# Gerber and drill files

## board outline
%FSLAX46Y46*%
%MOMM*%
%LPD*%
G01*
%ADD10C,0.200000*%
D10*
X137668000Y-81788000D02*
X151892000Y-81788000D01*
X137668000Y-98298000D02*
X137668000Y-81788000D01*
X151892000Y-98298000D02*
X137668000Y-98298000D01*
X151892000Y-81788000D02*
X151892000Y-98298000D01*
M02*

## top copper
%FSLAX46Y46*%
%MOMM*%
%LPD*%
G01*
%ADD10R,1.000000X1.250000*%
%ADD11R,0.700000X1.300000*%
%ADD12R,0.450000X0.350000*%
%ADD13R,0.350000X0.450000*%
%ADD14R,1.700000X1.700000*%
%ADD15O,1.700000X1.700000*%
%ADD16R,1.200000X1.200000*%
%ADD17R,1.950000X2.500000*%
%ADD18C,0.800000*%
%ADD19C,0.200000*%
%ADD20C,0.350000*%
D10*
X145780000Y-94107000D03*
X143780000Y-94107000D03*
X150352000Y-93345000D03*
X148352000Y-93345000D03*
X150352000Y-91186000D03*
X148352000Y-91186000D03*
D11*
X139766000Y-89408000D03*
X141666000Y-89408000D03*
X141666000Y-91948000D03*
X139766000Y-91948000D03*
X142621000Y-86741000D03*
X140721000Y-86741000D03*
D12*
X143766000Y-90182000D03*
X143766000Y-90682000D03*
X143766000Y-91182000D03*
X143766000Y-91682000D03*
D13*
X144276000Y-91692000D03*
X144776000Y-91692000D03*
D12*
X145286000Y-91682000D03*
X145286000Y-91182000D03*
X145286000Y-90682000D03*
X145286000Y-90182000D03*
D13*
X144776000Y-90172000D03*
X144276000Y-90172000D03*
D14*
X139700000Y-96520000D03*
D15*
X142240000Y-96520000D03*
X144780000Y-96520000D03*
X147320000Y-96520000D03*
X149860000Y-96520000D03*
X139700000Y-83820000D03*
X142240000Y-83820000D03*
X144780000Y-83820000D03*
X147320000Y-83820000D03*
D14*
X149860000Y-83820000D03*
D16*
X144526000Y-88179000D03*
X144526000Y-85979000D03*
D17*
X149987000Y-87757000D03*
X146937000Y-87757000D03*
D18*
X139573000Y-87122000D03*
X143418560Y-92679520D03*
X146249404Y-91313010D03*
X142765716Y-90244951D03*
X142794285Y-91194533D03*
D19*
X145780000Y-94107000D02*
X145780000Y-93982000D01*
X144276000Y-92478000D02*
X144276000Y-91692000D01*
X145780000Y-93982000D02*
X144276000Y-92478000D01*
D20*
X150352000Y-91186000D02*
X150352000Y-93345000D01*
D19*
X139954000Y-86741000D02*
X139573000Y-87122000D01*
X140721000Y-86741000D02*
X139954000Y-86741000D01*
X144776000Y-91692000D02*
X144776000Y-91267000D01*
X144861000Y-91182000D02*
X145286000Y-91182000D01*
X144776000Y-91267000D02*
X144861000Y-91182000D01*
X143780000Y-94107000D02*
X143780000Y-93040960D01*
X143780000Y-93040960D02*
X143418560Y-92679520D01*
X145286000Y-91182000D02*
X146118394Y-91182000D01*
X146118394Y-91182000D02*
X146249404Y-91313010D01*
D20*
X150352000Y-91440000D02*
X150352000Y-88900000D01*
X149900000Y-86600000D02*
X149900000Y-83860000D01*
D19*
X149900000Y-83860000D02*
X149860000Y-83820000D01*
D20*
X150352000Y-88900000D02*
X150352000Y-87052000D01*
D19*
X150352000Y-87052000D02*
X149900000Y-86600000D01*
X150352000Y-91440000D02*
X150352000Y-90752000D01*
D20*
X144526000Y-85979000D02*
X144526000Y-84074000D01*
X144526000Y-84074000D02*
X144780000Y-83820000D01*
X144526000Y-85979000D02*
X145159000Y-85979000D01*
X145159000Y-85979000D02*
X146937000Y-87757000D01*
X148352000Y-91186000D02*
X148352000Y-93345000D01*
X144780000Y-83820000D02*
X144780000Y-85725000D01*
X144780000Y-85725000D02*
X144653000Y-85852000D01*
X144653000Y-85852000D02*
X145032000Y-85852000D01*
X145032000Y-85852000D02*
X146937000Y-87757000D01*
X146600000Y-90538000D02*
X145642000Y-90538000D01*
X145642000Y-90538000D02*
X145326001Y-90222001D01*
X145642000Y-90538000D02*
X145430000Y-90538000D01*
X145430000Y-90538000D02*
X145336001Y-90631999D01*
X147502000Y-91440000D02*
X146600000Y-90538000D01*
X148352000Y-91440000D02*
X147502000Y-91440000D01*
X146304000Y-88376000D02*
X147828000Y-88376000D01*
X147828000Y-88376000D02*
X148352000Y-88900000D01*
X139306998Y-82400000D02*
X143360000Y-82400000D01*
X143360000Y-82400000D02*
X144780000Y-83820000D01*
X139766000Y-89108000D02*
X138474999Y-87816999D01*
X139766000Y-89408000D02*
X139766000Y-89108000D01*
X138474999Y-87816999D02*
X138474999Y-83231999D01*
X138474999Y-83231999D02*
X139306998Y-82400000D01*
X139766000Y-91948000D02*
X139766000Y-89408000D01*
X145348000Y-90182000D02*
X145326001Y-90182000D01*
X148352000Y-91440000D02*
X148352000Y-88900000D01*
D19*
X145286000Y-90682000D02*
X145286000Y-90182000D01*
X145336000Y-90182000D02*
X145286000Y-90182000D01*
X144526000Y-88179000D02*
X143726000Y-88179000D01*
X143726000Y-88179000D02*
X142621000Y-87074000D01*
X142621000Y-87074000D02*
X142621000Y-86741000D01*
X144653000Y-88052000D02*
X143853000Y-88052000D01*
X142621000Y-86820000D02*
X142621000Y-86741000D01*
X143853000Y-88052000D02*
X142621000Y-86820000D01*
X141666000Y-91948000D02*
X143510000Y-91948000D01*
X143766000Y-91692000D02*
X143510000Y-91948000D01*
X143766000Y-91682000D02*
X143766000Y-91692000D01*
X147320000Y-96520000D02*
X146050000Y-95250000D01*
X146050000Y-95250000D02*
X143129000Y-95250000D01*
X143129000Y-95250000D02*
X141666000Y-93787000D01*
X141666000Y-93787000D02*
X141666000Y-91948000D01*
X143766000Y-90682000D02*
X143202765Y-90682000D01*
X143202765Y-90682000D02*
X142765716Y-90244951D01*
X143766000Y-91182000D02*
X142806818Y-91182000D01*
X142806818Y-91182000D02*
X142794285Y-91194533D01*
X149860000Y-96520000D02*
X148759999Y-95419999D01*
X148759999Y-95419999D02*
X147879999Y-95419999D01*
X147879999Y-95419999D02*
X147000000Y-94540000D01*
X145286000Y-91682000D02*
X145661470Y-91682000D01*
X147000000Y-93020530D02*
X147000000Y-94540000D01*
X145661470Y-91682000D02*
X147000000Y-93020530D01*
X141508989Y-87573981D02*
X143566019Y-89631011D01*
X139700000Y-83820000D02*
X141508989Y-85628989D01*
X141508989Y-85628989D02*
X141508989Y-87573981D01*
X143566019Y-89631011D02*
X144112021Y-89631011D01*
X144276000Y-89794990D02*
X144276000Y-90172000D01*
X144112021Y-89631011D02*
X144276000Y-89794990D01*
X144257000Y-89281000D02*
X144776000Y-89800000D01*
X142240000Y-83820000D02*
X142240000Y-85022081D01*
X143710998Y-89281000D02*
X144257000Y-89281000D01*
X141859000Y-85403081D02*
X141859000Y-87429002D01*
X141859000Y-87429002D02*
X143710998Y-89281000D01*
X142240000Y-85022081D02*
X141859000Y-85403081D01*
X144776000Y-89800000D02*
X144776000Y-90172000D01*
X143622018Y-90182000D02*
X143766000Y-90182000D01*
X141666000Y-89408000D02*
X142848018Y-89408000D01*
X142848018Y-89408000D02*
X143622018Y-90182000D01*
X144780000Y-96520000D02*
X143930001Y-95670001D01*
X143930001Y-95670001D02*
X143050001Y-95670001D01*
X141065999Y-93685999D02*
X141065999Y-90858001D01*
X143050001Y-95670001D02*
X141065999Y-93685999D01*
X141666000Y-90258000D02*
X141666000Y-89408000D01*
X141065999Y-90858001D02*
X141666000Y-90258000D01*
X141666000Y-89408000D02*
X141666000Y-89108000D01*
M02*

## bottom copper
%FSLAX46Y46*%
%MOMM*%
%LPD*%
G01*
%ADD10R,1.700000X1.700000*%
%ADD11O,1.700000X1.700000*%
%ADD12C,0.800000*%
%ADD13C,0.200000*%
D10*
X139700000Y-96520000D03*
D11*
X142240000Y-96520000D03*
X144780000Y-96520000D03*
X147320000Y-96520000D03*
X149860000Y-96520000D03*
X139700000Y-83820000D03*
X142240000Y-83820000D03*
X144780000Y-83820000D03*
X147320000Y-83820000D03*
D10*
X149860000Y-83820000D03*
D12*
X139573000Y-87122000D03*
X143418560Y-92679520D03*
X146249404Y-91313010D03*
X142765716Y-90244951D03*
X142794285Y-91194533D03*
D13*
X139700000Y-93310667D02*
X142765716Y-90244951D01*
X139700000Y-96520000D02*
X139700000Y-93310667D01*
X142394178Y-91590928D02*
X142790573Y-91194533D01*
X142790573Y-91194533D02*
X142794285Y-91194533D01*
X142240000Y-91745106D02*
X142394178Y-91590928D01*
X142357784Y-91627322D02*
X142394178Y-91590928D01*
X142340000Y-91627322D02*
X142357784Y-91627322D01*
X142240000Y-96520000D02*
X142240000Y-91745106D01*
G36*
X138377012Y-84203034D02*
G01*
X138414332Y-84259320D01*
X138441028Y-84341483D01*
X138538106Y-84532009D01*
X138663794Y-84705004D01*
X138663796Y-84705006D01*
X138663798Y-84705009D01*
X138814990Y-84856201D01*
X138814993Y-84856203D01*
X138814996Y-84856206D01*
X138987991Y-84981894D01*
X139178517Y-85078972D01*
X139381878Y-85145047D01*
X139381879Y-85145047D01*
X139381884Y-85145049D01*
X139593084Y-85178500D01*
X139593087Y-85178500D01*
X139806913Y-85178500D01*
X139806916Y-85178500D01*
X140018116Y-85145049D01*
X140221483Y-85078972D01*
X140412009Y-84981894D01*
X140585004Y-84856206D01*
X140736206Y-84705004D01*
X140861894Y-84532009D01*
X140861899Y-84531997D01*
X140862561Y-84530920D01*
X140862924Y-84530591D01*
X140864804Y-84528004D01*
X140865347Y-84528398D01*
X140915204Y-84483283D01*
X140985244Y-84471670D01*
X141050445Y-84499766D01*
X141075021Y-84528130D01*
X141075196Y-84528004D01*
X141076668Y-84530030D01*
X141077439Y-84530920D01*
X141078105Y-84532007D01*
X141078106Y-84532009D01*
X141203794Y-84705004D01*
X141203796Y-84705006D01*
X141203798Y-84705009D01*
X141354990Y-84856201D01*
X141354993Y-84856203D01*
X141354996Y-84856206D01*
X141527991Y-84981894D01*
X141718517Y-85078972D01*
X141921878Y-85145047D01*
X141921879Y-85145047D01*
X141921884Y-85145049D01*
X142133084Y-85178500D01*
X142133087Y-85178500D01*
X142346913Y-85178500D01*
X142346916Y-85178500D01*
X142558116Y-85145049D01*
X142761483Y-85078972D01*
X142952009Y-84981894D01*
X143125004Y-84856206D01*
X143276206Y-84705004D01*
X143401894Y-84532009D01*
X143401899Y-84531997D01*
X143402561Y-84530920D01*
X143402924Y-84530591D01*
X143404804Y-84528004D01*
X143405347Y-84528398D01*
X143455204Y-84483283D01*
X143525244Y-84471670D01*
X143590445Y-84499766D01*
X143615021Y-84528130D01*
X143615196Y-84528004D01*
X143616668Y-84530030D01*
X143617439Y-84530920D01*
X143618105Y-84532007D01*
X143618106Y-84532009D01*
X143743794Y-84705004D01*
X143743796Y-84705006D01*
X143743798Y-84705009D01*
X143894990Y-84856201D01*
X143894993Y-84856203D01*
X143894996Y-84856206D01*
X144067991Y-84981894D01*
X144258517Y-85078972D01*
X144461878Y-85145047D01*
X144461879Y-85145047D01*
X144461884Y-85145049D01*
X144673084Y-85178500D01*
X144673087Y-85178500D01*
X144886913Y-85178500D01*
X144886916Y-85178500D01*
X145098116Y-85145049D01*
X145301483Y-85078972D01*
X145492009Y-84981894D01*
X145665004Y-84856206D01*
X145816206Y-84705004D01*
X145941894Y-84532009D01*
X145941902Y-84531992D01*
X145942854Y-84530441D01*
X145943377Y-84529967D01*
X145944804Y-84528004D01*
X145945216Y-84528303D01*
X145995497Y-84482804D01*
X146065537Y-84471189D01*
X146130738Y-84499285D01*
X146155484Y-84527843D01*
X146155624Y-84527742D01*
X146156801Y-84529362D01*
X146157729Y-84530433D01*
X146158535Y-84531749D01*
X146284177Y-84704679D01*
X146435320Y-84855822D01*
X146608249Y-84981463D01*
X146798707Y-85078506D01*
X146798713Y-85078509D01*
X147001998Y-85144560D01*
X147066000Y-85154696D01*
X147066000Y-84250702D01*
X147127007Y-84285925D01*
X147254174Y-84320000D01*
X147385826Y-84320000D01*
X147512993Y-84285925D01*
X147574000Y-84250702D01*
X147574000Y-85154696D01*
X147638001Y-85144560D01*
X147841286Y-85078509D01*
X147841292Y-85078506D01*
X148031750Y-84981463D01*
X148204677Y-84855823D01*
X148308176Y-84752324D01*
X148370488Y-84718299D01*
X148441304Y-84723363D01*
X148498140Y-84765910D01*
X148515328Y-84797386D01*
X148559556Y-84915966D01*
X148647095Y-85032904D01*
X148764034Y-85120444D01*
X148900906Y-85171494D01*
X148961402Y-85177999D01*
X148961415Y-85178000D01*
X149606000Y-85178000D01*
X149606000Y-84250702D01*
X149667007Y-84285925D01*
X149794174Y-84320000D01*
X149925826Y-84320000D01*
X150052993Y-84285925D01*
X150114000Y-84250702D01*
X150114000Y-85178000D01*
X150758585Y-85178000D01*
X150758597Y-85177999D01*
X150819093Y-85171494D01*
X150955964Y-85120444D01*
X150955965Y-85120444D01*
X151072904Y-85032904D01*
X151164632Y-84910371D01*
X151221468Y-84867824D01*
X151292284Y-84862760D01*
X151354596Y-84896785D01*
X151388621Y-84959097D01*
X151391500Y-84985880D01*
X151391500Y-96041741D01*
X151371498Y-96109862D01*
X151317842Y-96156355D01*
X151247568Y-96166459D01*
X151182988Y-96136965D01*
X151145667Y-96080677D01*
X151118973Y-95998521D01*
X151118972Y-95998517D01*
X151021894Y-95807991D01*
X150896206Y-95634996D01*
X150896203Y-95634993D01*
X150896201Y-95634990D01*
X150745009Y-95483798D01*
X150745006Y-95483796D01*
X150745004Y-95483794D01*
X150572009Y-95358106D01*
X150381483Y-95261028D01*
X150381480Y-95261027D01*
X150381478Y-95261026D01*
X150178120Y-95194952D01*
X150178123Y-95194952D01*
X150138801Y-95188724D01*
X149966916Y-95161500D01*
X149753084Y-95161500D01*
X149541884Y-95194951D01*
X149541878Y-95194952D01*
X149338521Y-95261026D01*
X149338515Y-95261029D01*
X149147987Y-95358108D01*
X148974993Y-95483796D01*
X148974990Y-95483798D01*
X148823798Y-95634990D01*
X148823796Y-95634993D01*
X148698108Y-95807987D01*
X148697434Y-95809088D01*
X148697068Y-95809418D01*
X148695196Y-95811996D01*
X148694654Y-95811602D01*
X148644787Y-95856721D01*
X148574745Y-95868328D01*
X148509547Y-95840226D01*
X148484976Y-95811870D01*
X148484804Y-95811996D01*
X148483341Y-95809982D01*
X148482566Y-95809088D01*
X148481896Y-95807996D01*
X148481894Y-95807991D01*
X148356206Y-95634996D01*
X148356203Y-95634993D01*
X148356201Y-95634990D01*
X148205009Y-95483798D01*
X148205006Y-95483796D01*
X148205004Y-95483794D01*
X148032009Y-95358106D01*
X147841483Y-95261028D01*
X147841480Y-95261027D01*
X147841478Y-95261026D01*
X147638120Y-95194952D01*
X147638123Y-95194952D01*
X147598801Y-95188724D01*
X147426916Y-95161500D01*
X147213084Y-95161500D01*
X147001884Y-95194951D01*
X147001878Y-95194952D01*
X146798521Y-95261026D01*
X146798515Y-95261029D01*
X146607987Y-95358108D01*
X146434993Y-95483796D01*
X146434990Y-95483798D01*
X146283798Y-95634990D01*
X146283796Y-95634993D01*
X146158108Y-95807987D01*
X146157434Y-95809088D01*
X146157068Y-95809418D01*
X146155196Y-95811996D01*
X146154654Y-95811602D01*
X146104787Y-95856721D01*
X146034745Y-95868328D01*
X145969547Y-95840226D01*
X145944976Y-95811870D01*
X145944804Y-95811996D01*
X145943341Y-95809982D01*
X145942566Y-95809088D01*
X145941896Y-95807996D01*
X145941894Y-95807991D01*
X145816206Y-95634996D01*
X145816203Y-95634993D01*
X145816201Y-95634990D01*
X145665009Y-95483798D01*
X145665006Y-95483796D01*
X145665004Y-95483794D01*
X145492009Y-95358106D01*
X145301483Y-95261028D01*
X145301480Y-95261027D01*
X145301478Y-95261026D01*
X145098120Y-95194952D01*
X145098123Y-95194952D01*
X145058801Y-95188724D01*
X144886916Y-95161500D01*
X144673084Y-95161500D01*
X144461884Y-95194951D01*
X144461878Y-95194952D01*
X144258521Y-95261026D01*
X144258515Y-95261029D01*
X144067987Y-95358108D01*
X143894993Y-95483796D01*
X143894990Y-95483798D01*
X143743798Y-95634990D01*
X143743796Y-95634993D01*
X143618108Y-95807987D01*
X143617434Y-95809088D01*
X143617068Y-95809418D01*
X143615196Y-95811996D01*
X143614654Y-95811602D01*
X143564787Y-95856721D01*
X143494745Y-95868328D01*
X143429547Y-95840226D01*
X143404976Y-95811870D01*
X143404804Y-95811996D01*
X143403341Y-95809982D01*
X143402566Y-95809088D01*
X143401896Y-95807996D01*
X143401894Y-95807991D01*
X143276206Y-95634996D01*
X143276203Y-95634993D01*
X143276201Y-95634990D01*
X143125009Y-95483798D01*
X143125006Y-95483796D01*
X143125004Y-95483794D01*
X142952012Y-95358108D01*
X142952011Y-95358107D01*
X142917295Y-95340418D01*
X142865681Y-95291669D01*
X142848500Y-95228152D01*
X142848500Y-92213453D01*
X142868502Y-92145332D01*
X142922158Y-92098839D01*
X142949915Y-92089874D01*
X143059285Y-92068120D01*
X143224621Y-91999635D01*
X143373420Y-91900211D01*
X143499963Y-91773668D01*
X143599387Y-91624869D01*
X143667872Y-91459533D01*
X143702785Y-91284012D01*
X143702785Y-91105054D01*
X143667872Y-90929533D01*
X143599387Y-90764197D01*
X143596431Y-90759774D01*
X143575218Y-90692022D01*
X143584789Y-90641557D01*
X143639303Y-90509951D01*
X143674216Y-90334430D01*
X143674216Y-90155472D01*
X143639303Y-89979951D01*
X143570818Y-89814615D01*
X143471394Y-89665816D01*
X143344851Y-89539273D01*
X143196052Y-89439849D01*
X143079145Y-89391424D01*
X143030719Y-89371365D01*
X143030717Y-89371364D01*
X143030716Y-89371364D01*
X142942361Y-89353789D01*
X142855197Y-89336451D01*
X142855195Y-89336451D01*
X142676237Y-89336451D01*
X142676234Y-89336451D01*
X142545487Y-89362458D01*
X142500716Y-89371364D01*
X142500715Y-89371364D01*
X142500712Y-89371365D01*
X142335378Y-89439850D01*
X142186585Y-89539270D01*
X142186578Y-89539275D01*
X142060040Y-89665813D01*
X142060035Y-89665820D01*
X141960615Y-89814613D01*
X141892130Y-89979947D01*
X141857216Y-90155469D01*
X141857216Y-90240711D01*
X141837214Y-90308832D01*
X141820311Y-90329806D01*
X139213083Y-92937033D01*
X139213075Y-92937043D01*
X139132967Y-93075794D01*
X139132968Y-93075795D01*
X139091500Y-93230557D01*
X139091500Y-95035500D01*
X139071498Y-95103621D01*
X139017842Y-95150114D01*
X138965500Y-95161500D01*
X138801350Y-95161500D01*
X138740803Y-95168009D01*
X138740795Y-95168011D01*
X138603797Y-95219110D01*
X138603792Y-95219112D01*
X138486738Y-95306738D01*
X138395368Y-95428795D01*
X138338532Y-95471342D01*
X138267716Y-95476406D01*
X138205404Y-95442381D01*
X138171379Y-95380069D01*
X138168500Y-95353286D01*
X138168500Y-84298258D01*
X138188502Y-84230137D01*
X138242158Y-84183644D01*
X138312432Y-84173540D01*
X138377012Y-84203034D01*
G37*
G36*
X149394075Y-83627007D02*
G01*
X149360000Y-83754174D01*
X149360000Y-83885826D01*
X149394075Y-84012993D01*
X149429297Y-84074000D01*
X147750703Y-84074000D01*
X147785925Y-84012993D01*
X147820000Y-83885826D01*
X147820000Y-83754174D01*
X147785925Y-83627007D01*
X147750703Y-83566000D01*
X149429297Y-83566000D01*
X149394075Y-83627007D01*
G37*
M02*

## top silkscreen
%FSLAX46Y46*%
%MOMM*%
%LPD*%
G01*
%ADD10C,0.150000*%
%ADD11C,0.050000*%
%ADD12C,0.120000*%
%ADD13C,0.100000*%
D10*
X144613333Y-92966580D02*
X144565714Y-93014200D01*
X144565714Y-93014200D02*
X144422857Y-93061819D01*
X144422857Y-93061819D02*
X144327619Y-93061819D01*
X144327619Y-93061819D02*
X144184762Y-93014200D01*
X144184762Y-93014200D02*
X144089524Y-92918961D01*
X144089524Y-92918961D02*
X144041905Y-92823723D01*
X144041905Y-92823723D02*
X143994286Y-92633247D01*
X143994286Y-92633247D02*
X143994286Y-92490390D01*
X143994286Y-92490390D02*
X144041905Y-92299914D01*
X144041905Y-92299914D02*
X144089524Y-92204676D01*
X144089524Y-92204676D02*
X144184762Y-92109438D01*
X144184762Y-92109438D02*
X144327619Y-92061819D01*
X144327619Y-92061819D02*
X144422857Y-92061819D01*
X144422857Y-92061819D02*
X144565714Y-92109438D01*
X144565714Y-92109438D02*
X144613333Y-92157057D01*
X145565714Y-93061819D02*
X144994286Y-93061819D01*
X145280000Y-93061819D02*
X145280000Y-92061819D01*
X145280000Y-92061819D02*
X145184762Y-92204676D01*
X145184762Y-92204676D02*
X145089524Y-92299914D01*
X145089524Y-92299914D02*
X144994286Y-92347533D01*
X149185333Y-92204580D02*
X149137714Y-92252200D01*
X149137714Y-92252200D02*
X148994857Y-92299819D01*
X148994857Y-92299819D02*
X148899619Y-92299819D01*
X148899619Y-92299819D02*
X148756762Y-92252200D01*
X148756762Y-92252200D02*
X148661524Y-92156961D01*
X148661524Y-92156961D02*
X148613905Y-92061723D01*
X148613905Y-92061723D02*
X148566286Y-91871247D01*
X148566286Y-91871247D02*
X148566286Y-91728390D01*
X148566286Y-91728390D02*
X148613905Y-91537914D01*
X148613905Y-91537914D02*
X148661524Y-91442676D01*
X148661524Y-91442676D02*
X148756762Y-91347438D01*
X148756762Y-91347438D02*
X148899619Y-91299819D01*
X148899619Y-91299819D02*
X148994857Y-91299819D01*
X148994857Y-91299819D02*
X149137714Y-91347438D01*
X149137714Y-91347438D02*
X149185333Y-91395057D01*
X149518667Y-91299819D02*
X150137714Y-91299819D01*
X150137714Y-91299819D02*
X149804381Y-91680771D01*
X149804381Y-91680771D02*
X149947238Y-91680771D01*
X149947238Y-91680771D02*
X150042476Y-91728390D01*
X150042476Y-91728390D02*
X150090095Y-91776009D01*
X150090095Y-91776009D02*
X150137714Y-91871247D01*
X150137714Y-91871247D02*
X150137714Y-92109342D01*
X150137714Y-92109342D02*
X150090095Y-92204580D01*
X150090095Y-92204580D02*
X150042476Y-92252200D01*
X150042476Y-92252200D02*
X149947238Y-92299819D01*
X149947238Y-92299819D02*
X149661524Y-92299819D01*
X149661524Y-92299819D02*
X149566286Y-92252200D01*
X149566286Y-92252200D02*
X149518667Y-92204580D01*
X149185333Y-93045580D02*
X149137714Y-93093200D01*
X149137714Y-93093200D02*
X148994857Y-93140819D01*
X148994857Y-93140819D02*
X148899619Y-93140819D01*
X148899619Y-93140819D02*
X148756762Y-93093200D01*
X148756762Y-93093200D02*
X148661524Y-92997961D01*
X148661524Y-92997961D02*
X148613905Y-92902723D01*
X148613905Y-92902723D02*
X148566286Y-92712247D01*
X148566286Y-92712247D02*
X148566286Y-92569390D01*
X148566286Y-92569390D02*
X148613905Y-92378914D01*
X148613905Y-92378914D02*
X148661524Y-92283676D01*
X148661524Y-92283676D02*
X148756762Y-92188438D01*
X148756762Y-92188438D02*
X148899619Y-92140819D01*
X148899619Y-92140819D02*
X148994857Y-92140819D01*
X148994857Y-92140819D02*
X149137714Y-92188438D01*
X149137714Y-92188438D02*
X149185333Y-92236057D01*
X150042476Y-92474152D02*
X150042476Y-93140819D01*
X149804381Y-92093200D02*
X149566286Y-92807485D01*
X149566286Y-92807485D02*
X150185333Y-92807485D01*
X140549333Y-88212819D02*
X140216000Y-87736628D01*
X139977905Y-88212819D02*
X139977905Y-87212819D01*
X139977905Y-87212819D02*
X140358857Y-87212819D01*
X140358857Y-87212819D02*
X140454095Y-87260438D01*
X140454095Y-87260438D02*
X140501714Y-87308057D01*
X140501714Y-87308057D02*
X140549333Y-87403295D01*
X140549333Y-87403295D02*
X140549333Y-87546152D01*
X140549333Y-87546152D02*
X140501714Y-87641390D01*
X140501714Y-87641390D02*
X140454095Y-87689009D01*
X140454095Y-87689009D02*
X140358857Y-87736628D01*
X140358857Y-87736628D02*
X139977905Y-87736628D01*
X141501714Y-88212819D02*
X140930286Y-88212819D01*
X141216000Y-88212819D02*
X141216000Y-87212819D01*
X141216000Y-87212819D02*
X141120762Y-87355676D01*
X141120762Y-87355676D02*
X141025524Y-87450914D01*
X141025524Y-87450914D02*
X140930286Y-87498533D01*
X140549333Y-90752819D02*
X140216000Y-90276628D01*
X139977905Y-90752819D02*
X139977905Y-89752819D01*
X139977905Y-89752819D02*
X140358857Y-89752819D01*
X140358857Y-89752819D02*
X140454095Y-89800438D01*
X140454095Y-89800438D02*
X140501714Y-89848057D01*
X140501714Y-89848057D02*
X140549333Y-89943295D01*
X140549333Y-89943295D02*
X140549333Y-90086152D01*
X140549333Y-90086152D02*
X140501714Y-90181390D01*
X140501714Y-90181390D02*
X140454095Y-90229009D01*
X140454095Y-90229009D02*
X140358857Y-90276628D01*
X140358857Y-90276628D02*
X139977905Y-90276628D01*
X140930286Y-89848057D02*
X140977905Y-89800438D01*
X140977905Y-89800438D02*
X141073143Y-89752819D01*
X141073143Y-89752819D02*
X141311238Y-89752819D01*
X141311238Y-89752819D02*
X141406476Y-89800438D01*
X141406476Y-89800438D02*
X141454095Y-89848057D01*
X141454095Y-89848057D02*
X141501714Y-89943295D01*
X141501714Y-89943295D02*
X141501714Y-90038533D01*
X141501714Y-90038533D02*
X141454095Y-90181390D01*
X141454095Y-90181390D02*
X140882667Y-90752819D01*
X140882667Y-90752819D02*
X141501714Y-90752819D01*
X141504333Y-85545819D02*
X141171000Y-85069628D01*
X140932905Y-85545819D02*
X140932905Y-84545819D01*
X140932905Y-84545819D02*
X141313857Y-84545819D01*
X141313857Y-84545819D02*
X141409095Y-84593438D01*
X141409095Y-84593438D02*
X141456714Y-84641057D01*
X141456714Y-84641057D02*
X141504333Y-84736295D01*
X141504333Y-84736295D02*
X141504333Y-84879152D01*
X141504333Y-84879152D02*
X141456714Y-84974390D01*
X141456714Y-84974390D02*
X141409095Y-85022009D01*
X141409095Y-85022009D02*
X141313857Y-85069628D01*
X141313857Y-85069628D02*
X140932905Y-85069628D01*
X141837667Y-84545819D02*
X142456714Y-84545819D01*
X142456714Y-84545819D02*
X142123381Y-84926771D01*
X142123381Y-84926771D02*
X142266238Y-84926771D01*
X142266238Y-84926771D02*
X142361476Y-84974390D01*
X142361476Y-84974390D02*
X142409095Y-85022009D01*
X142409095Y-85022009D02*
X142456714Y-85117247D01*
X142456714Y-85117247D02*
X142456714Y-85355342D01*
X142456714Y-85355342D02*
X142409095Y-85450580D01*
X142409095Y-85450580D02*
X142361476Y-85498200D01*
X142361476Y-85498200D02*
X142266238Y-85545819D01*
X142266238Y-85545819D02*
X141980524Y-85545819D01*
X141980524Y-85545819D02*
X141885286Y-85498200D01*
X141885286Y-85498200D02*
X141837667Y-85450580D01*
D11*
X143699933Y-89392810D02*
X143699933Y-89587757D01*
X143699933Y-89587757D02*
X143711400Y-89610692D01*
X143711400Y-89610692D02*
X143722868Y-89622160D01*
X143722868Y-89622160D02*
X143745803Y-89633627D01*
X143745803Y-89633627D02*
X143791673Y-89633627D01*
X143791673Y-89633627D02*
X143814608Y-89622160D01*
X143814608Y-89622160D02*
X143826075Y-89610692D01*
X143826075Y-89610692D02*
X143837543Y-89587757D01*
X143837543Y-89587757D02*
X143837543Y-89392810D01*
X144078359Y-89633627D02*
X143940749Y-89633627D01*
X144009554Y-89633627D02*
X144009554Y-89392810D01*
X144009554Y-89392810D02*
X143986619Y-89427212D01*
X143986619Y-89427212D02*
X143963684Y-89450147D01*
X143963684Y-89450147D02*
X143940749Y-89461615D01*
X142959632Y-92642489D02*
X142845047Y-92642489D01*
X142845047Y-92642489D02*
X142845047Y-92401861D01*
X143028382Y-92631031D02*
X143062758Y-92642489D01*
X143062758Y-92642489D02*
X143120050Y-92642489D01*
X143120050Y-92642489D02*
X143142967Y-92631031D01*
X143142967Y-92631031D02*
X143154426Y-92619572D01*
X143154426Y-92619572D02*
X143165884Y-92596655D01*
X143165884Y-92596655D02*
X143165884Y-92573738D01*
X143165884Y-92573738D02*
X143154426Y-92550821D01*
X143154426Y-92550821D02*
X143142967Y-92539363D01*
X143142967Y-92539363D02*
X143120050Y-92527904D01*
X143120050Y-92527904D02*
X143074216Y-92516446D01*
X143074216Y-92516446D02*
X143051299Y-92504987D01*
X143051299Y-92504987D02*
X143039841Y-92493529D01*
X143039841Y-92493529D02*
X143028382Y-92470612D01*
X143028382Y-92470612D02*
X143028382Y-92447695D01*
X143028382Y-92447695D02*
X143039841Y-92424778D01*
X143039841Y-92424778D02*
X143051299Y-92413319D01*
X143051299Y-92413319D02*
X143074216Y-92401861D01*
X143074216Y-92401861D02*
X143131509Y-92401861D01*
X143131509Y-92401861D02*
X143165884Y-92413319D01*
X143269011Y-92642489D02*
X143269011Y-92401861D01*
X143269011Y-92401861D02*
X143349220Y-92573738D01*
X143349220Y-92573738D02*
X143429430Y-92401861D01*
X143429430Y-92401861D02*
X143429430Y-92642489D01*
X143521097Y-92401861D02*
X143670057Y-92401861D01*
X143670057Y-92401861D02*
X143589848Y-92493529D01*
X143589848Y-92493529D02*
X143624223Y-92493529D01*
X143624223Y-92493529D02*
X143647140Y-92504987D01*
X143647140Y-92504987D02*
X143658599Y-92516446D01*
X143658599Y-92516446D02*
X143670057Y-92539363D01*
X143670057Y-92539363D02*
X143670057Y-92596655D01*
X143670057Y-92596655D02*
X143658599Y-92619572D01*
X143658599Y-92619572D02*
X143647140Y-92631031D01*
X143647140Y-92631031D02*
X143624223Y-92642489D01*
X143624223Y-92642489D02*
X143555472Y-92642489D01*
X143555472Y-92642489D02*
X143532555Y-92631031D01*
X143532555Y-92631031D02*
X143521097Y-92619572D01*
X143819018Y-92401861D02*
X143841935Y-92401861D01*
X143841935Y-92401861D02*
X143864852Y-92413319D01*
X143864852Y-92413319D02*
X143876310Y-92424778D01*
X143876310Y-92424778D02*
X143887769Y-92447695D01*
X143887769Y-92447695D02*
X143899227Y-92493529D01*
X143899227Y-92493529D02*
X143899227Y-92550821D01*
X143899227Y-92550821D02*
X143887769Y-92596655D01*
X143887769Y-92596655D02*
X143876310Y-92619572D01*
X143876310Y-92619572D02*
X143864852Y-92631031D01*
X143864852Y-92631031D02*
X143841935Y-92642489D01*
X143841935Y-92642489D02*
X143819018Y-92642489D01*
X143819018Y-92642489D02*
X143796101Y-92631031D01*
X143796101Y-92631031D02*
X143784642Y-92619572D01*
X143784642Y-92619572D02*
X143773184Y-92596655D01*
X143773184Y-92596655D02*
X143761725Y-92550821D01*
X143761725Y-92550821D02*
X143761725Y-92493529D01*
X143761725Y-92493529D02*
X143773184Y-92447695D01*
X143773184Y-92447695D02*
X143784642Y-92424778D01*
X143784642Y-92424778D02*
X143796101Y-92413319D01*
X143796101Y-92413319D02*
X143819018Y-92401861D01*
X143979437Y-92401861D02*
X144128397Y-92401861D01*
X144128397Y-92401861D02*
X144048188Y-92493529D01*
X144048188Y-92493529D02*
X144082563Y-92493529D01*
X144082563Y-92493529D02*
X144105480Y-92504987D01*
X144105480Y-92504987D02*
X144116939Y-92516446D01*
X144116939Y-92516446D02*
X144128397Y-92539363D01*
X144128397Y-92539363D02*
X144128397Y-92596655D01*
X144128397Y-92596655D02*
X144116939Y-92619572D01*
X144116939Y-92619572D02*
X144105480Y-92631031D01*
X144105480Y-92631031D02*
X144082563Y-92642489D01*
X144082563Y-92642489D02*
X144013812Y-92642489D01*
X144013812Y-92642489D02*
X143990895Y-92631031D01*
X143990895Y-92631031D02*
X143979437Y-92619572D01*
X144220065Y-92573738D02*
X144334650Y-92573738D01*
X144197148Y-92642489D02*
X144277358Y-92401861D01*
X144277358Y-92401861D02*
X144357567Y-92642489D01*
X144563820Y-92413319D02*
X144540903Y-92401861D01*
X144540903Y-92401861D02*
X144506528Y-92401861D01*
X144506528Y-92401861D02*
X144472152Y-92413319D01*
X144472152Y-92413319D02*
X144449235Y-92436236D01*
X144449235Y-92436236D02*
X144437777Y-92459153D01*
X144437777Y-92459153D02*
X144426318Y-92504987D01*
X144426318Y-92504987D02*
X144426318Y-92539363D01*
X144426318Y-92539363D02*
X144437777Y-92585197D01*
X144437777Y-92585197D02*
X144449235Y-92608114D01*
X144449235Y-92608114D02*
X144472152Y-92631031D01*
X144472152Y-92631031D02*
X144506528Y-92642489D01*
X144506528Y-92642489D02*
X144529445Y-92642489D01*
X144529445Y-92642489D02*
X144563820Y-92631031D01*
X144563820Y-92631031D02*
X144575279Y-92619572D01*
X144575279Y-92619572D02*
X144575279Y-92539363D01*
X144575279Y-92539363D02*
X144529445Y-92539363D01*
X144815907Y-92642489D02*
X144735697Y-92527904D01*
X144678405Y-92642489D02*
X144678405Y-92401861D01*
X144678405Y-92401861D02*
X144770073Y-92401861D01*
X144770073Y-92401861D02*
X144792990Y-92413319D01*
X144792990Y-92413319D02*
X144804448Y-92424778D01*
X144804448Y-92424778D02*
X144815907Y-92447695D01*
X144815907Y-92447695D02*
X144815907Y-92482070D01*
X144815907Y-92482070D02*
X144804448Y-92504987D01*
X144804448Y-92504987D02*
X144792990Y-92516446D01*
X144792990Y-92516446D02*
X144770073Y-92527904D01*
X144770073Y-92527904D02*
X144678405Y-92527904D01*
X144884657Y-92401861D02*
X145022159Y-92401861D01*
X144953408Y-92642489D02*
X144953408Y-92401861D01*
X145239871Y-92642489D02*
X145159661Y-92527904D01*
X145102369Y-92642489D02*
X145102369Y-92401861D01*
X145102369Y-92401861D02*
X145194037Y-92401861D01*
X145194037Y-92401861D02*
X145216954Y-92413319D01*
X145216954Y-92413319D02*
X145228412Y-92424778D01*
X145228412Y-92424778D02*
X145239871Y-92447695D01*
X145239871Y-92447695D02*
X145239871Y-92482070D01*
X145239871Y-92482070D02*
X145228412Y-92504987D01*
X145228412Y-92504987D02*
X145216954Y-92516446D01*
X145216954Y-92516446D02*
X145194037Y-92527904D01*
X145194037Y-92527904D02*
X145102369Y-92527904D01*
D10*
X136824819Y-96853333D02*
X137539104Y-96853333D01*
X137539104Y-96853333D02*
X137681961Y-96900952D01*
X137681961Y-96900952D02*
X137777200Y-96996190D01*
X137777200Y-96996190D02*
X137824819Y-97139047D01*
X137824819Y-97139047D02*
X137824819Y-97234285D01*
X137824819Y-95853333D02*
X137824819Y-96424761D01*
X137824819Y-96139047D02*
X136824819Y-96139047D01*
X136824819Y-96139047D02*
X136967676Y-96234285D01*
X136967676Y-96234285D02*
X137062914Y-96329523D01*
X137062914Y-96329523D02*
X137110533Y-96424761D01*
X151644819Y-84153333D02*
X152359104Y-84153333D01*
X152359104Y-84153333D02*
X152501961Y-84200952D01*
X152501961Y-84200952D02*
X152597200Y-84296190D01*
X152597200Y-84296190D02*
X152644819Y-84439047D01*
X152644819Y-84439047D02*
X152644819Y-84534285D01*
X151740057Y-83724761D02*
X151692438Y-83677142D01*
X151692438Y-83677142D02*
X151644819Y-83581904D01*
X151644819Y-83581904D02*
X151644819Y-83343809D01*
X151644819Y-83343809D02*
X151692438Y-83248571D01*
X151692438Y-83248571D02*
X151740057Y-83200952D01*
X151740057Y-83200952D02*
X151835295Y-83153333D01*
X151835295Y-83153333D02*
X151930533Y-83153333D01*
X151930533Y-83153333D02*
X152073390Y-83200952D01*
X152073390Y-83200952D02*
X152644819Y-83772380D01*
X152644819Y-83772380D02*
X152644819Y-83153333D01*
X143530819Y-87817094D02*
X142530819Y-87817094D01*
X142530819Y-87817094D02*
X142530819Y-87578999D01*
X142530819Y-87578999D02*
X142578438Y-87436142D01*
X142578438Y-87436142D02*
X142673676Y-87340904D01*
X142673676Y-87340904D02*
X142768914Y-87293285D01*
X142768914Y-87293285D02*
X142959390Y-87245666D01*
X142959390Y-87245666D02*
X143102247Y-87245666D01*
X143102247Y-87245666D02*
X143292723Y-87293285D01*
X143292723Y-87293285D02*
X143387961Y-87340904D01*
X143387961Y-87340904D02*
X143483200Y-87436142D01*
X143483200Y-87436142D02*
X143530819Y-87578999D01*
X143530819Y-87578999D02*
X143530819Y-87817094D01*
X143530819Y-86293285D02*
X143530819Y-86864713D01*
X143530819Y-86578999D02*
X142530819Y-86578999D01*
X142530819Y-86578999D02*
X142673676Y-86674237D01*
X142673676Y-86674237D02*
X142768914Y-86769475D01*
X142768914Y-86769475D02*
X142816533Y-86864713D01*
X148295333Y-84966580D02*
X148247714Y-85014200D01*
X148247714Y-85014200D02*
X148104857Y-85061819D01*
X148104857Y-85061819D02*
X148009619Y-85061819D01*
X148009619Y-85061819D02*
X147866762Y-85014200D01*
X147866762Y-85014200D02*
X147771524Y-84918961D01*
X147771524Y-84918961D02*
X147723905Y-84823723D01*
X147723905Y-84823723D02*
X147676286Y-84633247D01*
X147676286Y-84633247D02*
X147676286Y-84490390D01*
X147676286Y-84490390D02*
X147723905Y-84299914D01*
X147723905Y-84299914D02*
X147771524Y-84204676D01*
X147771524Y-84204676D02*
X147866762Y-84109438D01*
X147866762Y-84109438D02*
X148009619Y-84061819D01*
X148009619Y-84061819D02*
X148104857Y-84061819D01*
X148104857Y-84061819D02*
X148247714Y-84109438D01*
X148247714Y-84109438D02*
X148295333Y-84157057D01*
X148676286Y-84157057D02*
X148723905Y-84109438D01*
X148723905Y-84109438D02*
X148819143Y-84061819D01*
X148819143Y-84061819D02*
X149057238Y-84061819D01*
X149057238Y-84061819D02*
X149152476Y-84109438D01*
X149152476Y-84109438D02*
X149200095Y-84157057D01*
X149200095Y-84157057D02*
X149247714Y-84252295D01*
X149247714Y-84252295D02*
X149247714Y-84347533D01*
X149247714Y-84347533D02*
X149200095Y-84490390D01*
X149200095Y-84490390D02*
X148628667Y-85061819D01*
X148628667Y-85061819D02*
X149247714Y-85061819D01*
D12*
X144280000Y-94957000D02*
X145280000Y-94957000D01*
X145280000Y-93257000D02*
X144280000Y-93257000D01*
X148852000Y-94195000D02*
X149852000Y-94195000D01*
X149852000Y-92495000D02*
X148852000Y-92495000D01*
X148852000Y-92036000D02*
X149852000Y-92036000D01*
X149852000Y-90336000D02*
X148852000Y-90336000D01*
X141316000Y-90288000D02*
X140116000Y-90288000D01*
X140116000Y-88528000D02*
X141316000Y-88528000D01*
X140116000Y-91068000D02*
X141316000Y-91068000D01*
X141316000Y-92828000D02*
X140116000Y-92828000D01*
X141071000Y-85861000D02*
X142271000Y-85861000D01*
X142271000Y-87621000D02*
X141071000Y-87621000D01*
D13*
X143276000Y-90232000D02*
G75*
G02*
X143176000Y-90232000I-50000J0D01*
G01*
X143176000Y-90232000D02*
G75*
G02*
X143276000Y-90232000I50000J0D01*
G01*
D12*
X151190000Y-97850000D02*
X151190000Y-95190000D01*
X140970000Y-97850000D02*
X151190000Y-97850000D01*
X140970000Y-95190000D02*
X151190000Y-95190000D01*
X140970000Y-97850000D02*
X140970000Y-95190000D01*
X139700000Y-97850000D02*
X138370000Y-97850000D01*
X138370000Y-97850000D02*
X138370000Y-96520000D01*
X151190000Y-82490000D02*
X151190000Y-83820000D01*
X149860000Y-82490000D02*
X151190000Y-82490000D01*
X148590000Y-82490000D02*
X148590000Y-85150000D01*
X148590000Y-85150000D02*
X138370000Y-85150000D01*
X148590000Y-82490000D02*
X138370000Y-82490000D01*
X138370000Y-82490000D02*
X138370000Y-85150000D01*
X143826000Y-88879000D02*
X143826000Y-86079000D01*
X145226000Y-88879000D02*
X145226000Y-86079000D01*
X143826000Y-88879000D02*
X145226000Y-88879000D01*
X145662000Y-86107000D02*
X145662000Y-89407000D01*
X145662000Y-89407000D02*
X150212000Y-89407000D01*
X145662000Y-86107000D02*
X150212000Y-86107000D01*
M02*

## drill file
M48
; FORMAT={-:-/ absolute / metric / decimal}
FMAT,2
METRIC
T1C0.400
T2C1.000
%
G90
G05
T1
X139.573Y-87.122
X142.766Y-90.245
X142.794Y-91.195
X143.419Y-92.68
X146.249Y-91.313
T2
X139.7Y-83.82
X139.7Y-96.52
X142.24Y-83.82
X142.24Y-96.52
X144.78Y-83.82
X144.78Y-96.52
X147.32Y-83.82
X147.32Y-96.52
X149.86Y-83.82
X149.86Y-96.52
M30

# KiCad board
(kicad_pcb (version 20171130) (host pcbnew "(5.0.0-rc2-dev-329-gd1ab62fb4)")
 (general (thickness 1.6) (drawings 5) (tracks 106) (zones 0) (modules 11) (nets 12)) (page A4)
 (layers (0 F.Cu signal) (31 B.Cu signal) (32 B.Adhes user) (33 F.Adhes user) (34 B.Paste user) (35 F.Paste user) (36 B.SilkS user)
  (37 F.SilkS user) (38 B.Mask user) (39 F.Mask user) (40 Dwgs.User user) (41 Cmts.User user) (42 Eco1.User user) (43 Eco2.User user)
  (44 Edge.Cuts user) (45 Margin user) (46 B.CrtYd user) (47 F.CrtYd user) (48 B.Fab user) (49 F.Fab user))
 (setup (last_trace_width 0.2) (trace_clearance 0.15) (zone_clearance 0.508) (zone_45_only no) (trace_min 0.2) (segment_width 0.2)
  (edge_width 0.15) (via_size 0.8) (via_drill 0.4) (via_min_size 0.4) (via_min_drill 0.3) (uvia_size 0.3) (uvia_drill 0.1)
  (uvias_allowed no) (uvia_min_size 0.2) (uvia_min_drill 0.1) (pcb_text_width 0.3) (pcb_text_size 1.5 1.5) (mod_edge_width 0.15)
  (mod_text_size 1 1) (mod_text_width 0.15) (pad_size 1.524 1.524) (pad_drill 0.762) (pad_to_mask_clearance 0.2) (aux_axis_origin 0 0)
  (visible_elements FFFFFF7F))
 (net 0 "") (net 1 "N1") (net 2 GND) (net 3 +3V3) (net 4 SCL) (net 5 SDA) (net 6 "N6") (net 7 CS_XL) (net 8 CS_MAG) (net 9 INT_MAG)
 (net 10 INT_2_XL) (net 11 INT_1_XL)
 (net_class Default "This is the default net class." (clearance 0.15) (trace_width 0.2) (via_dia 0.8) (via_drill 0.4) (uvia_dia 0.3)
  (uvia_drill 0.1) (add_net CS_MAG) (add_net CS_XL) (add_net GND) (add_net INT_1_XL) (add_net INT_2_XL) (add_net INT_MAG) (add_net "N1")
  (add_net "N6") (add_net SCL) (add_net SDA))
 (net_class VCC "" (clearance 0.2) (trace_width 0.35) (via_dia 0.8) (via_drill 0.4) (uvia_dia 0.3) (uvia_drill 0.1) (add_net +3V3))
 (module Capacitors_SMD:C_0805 (layer F.Cu) (at 144.78 94.107)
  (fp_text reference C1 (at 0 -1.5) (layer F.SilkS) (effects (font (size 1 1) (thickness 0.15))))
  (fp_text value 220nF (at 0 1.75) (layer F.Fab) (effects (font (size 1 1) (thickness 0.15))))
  (fp_line (start -0.5 0.85) (end 0.5 0.85) (layer F.SilkS) (width 0.12))
  (fp_line (start 0.5 -0.85) (end -0.5 -0.85) (layer F.SilkS) (width 0.12))
  (pad 2 smd rect (at 1 0) (size 1 1.25) (layers F.Cu F.Paste F.Mask) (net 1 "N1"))
  (pad 1 smd rect (at -1 0) (size 1 1.25) (layers F.Cu F.Paste F.Mask) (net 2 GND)))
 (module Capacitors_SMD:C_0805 (layer F.Cu) (at 149.352 93.345)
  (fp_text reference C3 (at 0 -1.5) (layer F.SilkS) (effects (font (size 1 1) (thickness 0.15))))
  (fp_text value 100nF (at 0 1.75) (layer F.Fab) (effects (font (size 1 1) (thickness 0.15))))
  (fp_line (start -0.5 0.85) (end 0.5 0.85) (layer F.SilkS) (width 0.12))
  (fp_line (start 0.5 -0.85) (end -0.5 -0.85) (layer F.SilkS) (width 0.12))
  (pad 2 smd rect (at 1 0) (size 1 1.25) (layers F.Cu F.Paste F.Mask) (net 2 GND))
  (pad 1 smd rect (at -1 0) (size 1 1.25) (layers F.Cu F.Paste F.Mask) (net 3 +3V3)))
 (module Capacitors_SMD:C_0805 (layer F.Cu) (at 149.352 91.186 180)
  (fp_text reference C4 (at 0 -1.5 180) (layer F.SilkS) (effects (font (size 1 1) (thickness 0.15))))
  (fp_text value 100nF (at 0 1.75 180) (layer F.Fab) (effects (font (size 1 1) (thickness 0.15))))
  (fp_line (start 0.5 -0.85) (end -0.5 -0.85) (layer F.SilkS) (width 0.12))
  (fp_line (start -0.5 0.85) (end 0.5 0.85) (layer F.SilkS) (width 0.12))
  (pad 1 smd rect (at -1 0 180) (size 1 1.25) (layers F.Cu F.Paste F.Mask) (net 2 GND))
  (pad 2 smd rect (at 1 0 180) (size 1 1.25) (layers F.Cu F.Paste F.Mask) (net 3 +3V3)))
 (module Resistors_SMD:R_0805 (layer F.Cu) (at 140.716 89.408)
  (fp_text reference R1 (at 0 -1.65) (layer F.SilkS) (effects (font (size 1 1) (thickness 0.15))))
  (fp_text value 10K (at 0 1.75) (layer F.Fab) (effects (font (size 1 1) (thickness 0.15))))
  (fp_line (start 0.6 0.88) (end -0.6 0.88) (layer F.SilkS) (width 0.12))
  (fp_line (start -0.6 -0.88) (end 0.6 -0.88) (layer F.SilkS) (width 0.12))
  (pad 1 smd rect (at -0.95 0) (size 0.7 1.3) (layers F.Cu F.Paste F.Mask) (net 3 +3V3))
  (pad 2 smd rect (at 0.95 0) (size 0.7 1.3) (layers F.Cu F.Paste F.Mask) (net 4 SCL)))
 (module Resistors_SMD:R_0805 (layer F.Cu) (at 140.716 91.948)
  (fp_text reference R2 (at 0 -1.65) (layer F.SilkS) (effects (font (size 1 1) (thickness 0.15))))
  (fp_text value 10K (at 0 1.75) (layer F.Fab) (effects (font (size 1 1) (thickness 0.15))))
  (fp_line (start -0.6 -0.88) (end 0.6 -0.88) (layer F.SilkS) (width 0.12))
  (fp_line (start 0.6 0.88) (end -0.6 0.88) (layer F.SilkS) (width 0.12))
  (pad 2 smd rect (at 0.95 0) (size 0.7 1.3) (layers F.Cu F.Paste F.Mask) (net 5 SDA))
  (pad 1 smd rect (at -0.95 0) (size 0.7 1.3) (layers F.Cu F.Paste F.Mask) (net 3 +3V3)))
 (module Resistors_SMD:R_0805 (layer F.Cu) (at 141.671 86.741)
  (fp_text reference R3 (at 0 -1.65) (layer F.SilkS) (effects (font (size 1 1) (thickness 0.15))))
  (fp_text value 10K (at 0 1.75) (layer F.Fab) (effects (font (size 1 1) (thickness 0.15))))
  (fp_line (start -0.6 -0.88) (end 0.6 -0.88) (layer F.SilkS) (width 0.12))
  (fp_line (start 0.6 0.88) (end -0.6 0.88) (layer F.SilkS) (width 0.12))
  (pad 2 smd rect (at 0.95 0) (size 0.7 1.3) (layers F.Cu F.Paste F.Mask) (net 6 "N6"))
  (pad 1 smd rect (at -0.95 0) (size 0.7 1.3) (layers F.Cu F.Paste F.Mask) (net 2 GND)))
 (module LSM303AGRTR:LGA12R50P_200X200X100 (layer F.Cu) (at 144.526 90.932)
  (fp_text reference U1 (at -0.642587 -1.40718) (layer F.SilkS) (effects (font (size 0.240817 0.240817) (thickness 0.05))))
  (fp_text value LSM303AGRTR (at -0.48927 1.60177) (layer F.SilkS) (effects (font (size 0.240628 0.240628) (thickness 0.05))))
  (fp_circle (center -1.3 -0.7) (end -1.2 -0.7) (layer F.SilkS) (width 0))
  (pad 1 smd rect (at -0.76 -0.75) (size 0.45 0.35) (layers F.Cu F.Paste F.Mask) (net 4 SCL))
  (pad 2 smd rect (at -0.76 -0.25) (size 0.45 0.35) (layers F.Cu F.Paste F.Mask) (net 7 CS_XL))
  (pad 3 smd rect (at -0.76 0.25) (size 0.45 0.35) (layers F.Cu F.Paste F.Mask) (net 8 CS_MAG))
  (pad 4 smd rect (at -0.76 0.75) (size 0.45 0.35) (layers F.Cu F.Paste F.Mask) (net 5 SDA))
  (pad 5 smd rect (at -0.25 0.76 90) (size 0.45 0.35) (layers F.Cu F.Paste F.Mask) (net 1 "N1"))
  (pad 6 smd rect (at 0.25 0.76 90) (size 0.45 0.35) (layers F.Cu F.Paste F.Mask) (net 2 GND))
  (pad 7 smd rect (at 0.76 0.75) (size 0.45 0.35) (layers F.Cu F.Paste F.Mask) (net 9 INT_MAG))
  (pad 8 smd rect (at 0.76 0.25) (size 0.45 0.35) (layers F.Cu F.Paste F.Mask) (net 2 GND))
  (pad 9 smd rect (at 0.76 -0.25) (size 0.45 0.35) (layers F.Cu F.Paste F.Mask) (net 3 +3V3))
  (pad 10 smd rect (at 0.76 -0.75) (size 0.45 0.35) (layers F.Cu F.Paste F.Mask) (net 3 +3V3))
  (pad 11 smd rect (at 0.25 -0.76 90) (size 0.45 0.35) (layers F.Cu F.Paste F.Mask) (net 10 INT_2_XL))
  (pad 12 smd rect (at -0.25 -0.76 90) (size 0.45 0.35) (layers F.Cu F.Paste F.Mask) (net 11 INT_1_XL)))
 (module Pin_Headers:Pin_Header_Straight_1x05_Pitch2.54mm (layer F.Cu) (at 139.7 96.52 90)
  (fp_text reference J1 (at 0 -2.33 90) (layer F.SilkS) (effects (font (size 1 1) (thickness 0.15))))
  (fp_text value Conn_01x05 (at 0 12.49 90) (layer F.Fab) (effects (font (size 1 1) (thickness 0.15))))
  (fp_line (start -1.33 11.49) (end 1.33 11.49) (layer F.SilkS) (width 0.12))
  (fp_line (start -1.33 1.27) (end -1.33 11.49) (layer F.SilkS) (width 0.12))
  (fp_line (start 1.33 1.27) (end 1.33 11.49) (layer F.SilkS) (width 0.12))
  (fp_line (start -1.33 1.27) (end 1.33 1.27) (layer F.SilkS) (width 0.12))
  (fp_line (start -1.33 0) (end -1.33 -1.33) (layer F.SilkS) (width 0.12))
  (fp_line (start -1.33 -1.33) (end 0 -1.33) (layer F.SilkS) (width 0.12))
  (pad 1 thru_hole rect (at 0 0 90) (size 1.7 1.7) (drill 1) (layers *.Cu *.Mask) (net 7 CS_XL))
  (pad 2 thru_hole oval (at 0 2.54 90) (size 1.7 1.7) (drill 1) (layers *.Cu *.Mask) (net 8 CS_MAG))
  (pad 3 thru_hole oval (at 0 5.08 90) (size 1.7 1.7) (drill 1) (layers *.Cu *.Mask) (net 4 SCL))
  (pad 4 thru_hole oval (at 0 7.62 90) (size 1.7 1.7) (drill 1) (layers *.Cu *.Mask) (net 5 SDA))
  (pad 5 thru_hole oval (at 0 10.16 90) (size 1.7 1.7) (drill 1) (layers *.Cu *.Mask) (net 9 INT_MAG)))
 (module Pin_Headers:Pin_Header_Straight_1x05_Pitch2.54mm (layer F.Cu) (at 149.86 83.82 270)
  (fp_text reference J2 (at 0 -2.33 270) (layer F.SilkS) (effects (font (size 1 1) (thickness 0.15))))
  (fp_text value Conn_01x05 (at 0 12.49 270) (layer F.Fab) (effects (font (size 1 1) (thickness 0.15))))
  (fp_line (start -1.33 -1.33) (end 0 -1.33) (layer F.SilkS) (width 0.12))
  (fp_line (start -1.33 0) (end -1.33 -1.33) (layer F.SilkS) (width 0.12))
  (fp_line (start -1.33 1.27) (end 1.33 1.27) (layer F.SilkS) (width 0.12))
  (fp_line (start 1.33 1.27) (end 1.33 11.49) (layer F.SilkS) (width 0.12))
  (fp_line (start -1.33 1.27) (end -1.33 11.49) (layer F.SilkS) (width 0.12))
  (fp_line (start -1.33 11.49) (end 1.33 11.49) (layer F.SilkS) (width 0.12))
  (pad 5 thru_hole oval (at 0 10.16 270) (size 1.7 1.7) (drill 1) (layers *.Cu *.Mask) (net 11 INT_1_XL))
  (pad 4 thru_hole oval (at 0 7.62 270) (size 1.7 1.7) (drill 1) (layers *.Cu *.Mask) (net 10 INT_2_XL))
  (pad 3 thru_hole oval (at 0 5.08 270) (size 1.7 1.7) (drill 1) (layers *.Cu *.Mask) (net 3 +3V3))
  (pad 2 thru_hole oval (at 0 2.54 270) (size 1.7 1.7) (drill 1) (layers *.Cu *.Mask) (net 2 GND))
  (pad 1 thru_hole rect (at 0 0 270) (size 1.7 1.7) (drill 1) (layers *.Cu *.Mask) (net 2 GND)))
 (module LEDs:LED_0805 (layer F.Cu) (at 144.526 87.079 90)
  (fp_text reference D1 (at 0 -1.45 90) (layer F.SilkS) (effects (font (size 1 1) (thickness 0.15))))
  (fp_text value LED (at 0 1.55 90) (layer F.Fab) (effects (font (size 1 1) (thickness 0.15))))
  (fp_line (start -1.8 -0.7) (end 1 -0.7) (layer F.SilkS) (width 0.12))
  (fp_line (start -1.8 0.7) (end 1 0.7) (layer F.SilkS) (width 0.12))
  (fp_line (start -1.8 -0.7) (end -1.8 0.7) (layer F.SilkS) (width 0.12))
  (pad 1 smd rect (at -1.1 0 270) (size 1.2 1.2) (layers F.Cu F.Paste F.Mask) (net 6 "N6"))
  (pad 2 smd rect (at 1.1 0 270) (size 1.2 1.2) (layers F.Cu F.Paste F.Mask) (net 3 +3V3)))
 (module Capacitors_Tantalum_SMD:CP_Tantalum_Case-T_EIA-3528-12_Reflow (layer F.Cu) (at 148.462 87.757)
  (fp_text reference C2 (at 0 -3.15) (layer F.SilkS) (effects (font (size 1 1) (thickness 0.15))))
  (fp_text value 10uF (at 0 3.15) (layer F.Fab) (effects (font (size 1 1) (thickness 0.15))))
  (fp_line (start -2.8 -1.65) (end -2.8 1.65) (layer F.SilkS) (width 0.12))
  (fp_line (start -2.8 1.65) (end 1.75 1.65) (layer F.SilkS) (width 0.12))
  (fp_line (start -2.8 -1.65) (end 1.75 -1.65) (layer F.SilkS) (width 0.12))
  (pad 2 smd rect (at 1.525 0) (size 1.95 2.5) (layers F.Cu F.Paste F.Mask) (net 2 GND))
  (pad 1 smd rect (at -1.525 0) (size 1.95 2.5) (layers F.Cu F.Paste F.Mask) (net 3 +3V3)))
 (gr_line (start 137.668 81.788) (end 151.892 81.788) (layer Edge.Cuts) (width 0.2))
 (gr_line (start 137.668 98.298) (end 137.668 81.788) (layer Edge.Cuts) (width 0.2))
 (gr_line (start 151.892 98.298) (end 137.668 98.298) (layer Edge.Cuts) (width 0.2))
 (gr_line (start 151.892 81.788) (end 151.892 98.298) (layer Edge.Cuts) (width 0.2))
 (segment (start 145.78 94.107) (end 145.78 93.982) (width 0.2) (layer F.Cu) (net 1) (status 30))
 (segment (start 144.276 92.478) (end 144.276 91.692) (width 0.2) (layer F.Cu) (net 1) (status 20))
 (segment (start 145.78 93.982) (end 144.276 92.478) (width 0.2) (layer F.Cu) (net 1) (status 10))
 (segment (start 150.352 91.186) (end 150.352 93.345) (width 0.35) (layer F.Cu) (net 2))
 (segment (start 139.954 86.741) (end 139.573 87.122) (width 0.2) (layer F.Cu) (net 2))
 (segment (start 140.721 86.741) (end 139.954 86.741) (width 0.2) (layer F.Cu) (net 2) (status 10))
 (via (at 139.573 87.122) (size 0.8) (drill 0.4) (layers F.Cu B.Cu) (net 2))
 (segment (start 144.776 91.692) (end 144.776 91.267) (width 0.2) (layer F.Cu) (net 2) (status 10))
 (segment (start 144.861 91.182) (end 145.286 91.182) (width 0.2) (layer F.Cu) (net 2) (status 20))
 (segment (start 144.776 91.267) (end 144.861 91.182) (width 0.2) (layer F.Cu) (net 2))
 (segment (start 143.78 94.107) (end 143.78 93.04096) (width 0.2) (layer F.Cu) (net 2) (status 10))
 (segment (start 143.78 93.04096) (end 143.41856 92.67952) (width 0.2) (layer F.Cu) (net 2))
 (via (at 143.41856 92.67952) (size 0.8) (drill 0.4) (layers F.Cu B.Cu) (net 2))
 (via (at 146.249404 91.31301) (size 0.8) (drill 0.4) (layers F.Cu B.Cu) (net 2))
 (segment (start 145.286 91.182) (end 146.118394 91.182) (width 0.2) (layer F.Cu) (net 2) (status 10))
 (segment (start 146.118394 91.182) (end 146.249404 91.31301) (width 0.2) (layer F.Cu) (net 2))
 (segment (start 150.352 91.44) (end 150.352 88.9) (width 0.35) (layer F.Cu) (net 2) (status 30))
 (segment (start 149.9 86.6) (end 149.9 83.86) (width 0.35) (layer F.Cu) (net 2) (status 30))
 (segment (start 149.9 83.86) (end 149.86 83.82) (width 0.2) (layer F.Cu) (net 2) (status 30))
 (segment (start 150.352 88.9) (end 150.352 87.052) (width 0.35) (layer F.Cu) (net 2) (status 30))
 (segment (start 150.352 87.052) (end 149.9 86.6) (width 0.2) (layer F.Cu) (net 2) (status 30))
 (segment (start 150.352 91.44) (end 150.352 90.752) (width 0.2) (layer F.Cu) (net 2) (status 30))
 (segment (start 144.526 85.979) (end 144.526 84.074) (width 0.35) (layer F.Cu) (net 3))
 (segment (start 144.526 84.074) (end 144.78 83.82) (width 0.35) (layer F.Cu) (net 3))
 (segment (start 144.526 85.979) (end 145.159 85.979) (width 0.35) (layer F.Cu) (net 3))
 (segment (start 145.159 85.979) (end 146.937 87.757) (width 0.35) (layer F.Cu) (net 3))
 (segment (start 148.352 91.186) (end 148.352 93.345) (width 0.35) (layer F.Cu) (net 3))
 (segment (start 144.78 83.82) (end 144.78 85.725) (width 0.35) (layer F.Cu) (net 3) (status 30))
 (segment (start 144.78 85.725) (end 144.653 85.852) (width 0.35) (layer F.Cu) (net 3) (status 30))
 (segment (start 144.653 85.852) (end 145.032 85.852) (width 0.35) (layer F.Cu) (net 3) (status 30))
 (segment (start 145.032 85.852) (end 146.937 87.757) (width 0.35) (layer F.Cu) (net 3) (status 30))
 (segment (start 146.6 90.538) (end 145.642 90.538) (width 0.35) (layer F.Cu) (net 3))
 (segment (start 145.642 90.538) (end 145.326001 90.222001) (width 0.35) (layer F.Cu) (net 3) (status 20))
 (segment (start 145.642 90.538) (end 145.43 90.538) (width 0.35) (layer F.Cu) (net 3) (status 20))
 (segment (start 145.43 90.538) (end 145.336001 90.631999) (width 0.35) (layer F.Cu) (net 3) (status 30))
 (segment (start 147.502 91.44) (end 146.6 90.538) (width 0.35) (layer F.Cu) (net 3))
 (segment (start 148.352 91.44) (end 147.502 91.44) (width 0.35) (layer F.Cu) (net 3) (status 10))
 (segment (start 146.304 88.376) (end 147.828 88.376) (width 0.35) (layer F.Cu) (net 3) (status 30))
 (segment (start 147.828 88.376) (end 148.352 88.9) (width 0.35) (layer F.Cu) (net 3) (status 10))
 (segment (start 139.306998 82.4) (end 143.36 82.4) (width 0.35) (layer F.Cu) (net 3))
 (segment (start 143.36 82.4) (end 144.78 83.82) (width 0.35) (layer F.Cu) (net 3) (status 20))
 (segment (start 139.766 89.108) (end 138.474999 87.816999) (width 0.35) (layer F.Cu) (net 3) (status 10))
 (segment (start 139.766 89.408) (end 139.766 89.108) (width 0.35) (layer F.Cu) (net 3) (status 30))
 (segment (start 138.474999 87.816999) (end 138.474999 83.231999) (width 0.35) (layer F.Cu) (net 3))
 (segment (start 138.474999 83.231999) (end 139.306998 82.4) (width 0.35) (layer F.Cu) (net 3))
 (segment (start 139.766 91.948) (end 139.766 89.408) (width 0.35) (layer F.Cu) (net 3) (status 30))
 (segment (start 145.348 90.182) (end 145.326001 90.182) (width 0.35) (layer F.Cu) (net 3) (status 30))
 (segment (start 148.352 91.44) (end 148.352 88.9) (width 0.35) (layer F.Cu) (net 3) (status 10))
 (segment (start 145.286 90.682) (end 145.286 90.182) (width 0.2) (layer F.Cu) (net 3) (status 30))
 (segment (start 145.336 90.182) (end 145.286 90.182) (width 0.2) (layer F.Cu) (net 3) (status 30))
 (segment (start 144.526 88.179) (end 143.726 88.179) (width 0.2) (layer F.Cu) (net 6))
 (segment (start 143.726 88.179) (end 142.621 87.074) (width 0.2) (layer F.Cu) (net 6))
 (segment (start 142.621 87.074) (end 142.621 86.741) (width 0.2) (layer F.Cu) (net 6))
 (segment (start 144.653 88.052) (end 143.853 88.052) (width 0.2) (layer F.Cu) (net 6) (status 10))
 (segment (start 142.621 86.82) (end 142.621 86.741) (width 0.2) (layer F.Cu) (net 6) (status 30))
 (segment (start 143.853 88.052) (end 142.621 86.82) (width 0.2) (layer F.Cu) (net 6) (status 20))
 (segment (start 141.666 91.948) (end 143.51 91.948) (width 0.2) (layer F.Cu) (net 5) (status 10))
 (segment (start 143.766 91.692) (end 143.51 91.948) (width 0.2) (layer F.Cu) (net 5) (status 10))
 (segment (start 143.766 91.682) (end 143.766 91.692) (width 0.2) (layer F.Cu) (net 5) (status 30))
 (segment (start 147.32 96.52) (end 146.05 95.25) (width 0.2) (layer F.Cu) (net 5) (status 10))
 (segment (start 146.05 95.25) (end 143.129 95.25) (width 0.2) (layer F.Cu) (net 5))
 (segment (start 143.129 95.25) (end 141.666 93.787) (width 0.2) (layer F.Cu) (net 5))
 (segment (start 141.666 93.787) (end 141.666 91.948) (width 0.2) (layer F.Cu) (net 5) (status 20))
 (segment (start 139.7 93.310667) (end 142.765716 90.244951) (width 0.2) (layer B.Cu) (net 7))
 (segment (start 143.766 90.682) (end 143.202765 90.682) (width 0.2) (layer F.Cu) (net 7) (status 10))
 (segment (start 139.7 96.52) (end 139.7 93.310667) (width 0.2) (layer B.Cu) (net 7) (status 10))
 (segment (start 143.202765 90.682) (end 142.765716 90.244951) (width 0.2) (layer F.Cu) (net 7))
 (via (at 142.765716 90.244951) (size 0.8) (drill 0.4) (layers F.Cu B.Cu) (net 7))
 (segment (start 143.766 91.182) (end 142.806818 91.182) (width 0.2) (layer F.Cu) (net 8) (status 10))
 (segment (start 142.394178 91.590928) (end 142.790573 91.194533) (width 0.2) (layer B.Cu) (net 8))
 (segment (start 142.790573 91.194533) (end 142.794285 91.194533) (width 0.2) (layer B.Cu) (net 8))
 (segment (start 142.806818 91.182) (end 142.794285 91.194533) (width 0.2) (layer F.Cu) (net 8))
 (via (at 142.794285 91.194533) (size 0.8) (drill 0.4) (layers F.Cu B.Cu) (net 8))
 (segment (start 142.24 91.745106) (end 142.394178 91.590928) (width 0.2) (layer B.Cu) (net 8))
 (segment (start 142.357784 91.627322) (end 142.394178 91.590928) (width 0.2) (layer B.Cu) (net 8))
 (segment (start 142.34 91.627322) (end 142.357784 91.627322) (width 0.2) (layer B.Cu) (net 8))
 (segment (start 142.24 96.52) (end 142.24 91.745106) (width 0.2) (layer B.Cu) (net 8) (status 10))
 (segment (start 149.86 96.52) (end 148.759999 95.419999) (width 0.2) (layer F.Cu) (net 9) (status 10))
 (segment (start 148.759999 95.419999) (end 147.879999 95.419999) (width 0.2) (layer F.Cu) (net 9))
 (segment (start 147.879999 95.419999) (end 147 94.54) (width 0.2) (layer F.Cu) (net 9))
 (segment (start 145.286 91.682) (end 145.66147 91.682) (width 0.2) (layer F.Cu) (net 9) (status 10))
 (segment (start 147 93.02053) (end 147 94.54) (width 0.2) (layer F.Cu) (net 9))
 (segment (start 145.66147 91.682) (end 147 93.02053) (width 0.2) (layer F.Cu) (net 9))
 (segment (start 141.508989 87.573981) (end 143.566019 89.631011) (width 0.2) (layer F.Cu) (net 11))
 (segment (start 139.7 83.82) (end 141.508989 85.628989) (width 0.2) (layer F.Cu) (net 11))
 (segment (start 141.508989 85.628989) (end 141.508989 87.573981) (width 0.2) (layer F.Cu) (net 11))
 (segment (start 143.566019 89.631011) (end 144.112021 89.631011) (width 0.2) (layer F.Cu) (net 11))
 (segment (start 144.276 89.79499) (end 144.276 90.172) (width 0.2) (layer F.Cu) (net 11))
 (segment (start 144.112021 89.631011) (end 144.276 89.79499) (width 0.2) (layer F.Cu) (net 11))
 (segment (start 144.257 89.281) (end 144.776 89.8) (width 0.2) (layer F.Cu) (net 10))
 (segment (start 142.24 83.82) (end 142.24 85.022081) (width 0.2) (layer F.Cu) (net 10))
 (segment (start 143.710998 89.281) (end 144.257 89.281) (width 0.2) (layer F.Cu) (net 10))
 (segment (start 141.859 85.403081) (end 141.859 87.429002) (width 0.2) (layer F.Cu) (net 10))
 (segment (start 141.859 87.429002) (end 143.710998 89.281) (width 0.2) (layer F.Cu) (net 10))
 (segment (start 142.24 85.022081) (end 141.859 85.403081) (width 0.2) (layer F.Cu) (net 10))
 (segment (start 144.776 89.8) (end 144.776 90.172) (width 0.2) (layer F.Cu) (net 10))
 (segment (start 143.622018 90.182) (end 143.766 90.182) (width 0.2) (layer F.Cu) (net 4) (status 30))
 (segment (start 141.666 89.408) (end 142.848018 89.408) (width 0.2) (layer F.Cu) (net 4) (status 10))
 (segment (start 142.848018 89.408) (end 143.622018 90.182) (width 0.2) (layer F.Cu) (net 4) (status 20))
 (segment (start 144.78 96.52) (end 143.930001 95.670001) (width 0.2) (layer F.Cu) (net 4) (status 10))
 (segment (start 143.930001 95.670001) (end 143.050001 95.670001) (width 0.2) (layer F.Cu) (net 4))
 (segment (start 141.065999 93.685999) (end 141.065999 90.858001) (width 0.2) (layer F.Cu) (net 4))
 (segment (start 143.050001 95.670001) (end 141.065999 93.685999) (width 0.2) (layer F.Cu) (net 4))
 (segment (start 141.666 90.258) (end 141.666 89.408) (width 0.2) (layer F.Cu) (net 4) (status 20))
 (segment (start 141.065999 90.858001) (end 141.666 90.258) (width 0.2) (layer F.Cu) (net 4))
 (segment (start 141.666 89.408) (end 141.666 89.108) (width 0.2) (layer F.Cu) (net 4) (status 30))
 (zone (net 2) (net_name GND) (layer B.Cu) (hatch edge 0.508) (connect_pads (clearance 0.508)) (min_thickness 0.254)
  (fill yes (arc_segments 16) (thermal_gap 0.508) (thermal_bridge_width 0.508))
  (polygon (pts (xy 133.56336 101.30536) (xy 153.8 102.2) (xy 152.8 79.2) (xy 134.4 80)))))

